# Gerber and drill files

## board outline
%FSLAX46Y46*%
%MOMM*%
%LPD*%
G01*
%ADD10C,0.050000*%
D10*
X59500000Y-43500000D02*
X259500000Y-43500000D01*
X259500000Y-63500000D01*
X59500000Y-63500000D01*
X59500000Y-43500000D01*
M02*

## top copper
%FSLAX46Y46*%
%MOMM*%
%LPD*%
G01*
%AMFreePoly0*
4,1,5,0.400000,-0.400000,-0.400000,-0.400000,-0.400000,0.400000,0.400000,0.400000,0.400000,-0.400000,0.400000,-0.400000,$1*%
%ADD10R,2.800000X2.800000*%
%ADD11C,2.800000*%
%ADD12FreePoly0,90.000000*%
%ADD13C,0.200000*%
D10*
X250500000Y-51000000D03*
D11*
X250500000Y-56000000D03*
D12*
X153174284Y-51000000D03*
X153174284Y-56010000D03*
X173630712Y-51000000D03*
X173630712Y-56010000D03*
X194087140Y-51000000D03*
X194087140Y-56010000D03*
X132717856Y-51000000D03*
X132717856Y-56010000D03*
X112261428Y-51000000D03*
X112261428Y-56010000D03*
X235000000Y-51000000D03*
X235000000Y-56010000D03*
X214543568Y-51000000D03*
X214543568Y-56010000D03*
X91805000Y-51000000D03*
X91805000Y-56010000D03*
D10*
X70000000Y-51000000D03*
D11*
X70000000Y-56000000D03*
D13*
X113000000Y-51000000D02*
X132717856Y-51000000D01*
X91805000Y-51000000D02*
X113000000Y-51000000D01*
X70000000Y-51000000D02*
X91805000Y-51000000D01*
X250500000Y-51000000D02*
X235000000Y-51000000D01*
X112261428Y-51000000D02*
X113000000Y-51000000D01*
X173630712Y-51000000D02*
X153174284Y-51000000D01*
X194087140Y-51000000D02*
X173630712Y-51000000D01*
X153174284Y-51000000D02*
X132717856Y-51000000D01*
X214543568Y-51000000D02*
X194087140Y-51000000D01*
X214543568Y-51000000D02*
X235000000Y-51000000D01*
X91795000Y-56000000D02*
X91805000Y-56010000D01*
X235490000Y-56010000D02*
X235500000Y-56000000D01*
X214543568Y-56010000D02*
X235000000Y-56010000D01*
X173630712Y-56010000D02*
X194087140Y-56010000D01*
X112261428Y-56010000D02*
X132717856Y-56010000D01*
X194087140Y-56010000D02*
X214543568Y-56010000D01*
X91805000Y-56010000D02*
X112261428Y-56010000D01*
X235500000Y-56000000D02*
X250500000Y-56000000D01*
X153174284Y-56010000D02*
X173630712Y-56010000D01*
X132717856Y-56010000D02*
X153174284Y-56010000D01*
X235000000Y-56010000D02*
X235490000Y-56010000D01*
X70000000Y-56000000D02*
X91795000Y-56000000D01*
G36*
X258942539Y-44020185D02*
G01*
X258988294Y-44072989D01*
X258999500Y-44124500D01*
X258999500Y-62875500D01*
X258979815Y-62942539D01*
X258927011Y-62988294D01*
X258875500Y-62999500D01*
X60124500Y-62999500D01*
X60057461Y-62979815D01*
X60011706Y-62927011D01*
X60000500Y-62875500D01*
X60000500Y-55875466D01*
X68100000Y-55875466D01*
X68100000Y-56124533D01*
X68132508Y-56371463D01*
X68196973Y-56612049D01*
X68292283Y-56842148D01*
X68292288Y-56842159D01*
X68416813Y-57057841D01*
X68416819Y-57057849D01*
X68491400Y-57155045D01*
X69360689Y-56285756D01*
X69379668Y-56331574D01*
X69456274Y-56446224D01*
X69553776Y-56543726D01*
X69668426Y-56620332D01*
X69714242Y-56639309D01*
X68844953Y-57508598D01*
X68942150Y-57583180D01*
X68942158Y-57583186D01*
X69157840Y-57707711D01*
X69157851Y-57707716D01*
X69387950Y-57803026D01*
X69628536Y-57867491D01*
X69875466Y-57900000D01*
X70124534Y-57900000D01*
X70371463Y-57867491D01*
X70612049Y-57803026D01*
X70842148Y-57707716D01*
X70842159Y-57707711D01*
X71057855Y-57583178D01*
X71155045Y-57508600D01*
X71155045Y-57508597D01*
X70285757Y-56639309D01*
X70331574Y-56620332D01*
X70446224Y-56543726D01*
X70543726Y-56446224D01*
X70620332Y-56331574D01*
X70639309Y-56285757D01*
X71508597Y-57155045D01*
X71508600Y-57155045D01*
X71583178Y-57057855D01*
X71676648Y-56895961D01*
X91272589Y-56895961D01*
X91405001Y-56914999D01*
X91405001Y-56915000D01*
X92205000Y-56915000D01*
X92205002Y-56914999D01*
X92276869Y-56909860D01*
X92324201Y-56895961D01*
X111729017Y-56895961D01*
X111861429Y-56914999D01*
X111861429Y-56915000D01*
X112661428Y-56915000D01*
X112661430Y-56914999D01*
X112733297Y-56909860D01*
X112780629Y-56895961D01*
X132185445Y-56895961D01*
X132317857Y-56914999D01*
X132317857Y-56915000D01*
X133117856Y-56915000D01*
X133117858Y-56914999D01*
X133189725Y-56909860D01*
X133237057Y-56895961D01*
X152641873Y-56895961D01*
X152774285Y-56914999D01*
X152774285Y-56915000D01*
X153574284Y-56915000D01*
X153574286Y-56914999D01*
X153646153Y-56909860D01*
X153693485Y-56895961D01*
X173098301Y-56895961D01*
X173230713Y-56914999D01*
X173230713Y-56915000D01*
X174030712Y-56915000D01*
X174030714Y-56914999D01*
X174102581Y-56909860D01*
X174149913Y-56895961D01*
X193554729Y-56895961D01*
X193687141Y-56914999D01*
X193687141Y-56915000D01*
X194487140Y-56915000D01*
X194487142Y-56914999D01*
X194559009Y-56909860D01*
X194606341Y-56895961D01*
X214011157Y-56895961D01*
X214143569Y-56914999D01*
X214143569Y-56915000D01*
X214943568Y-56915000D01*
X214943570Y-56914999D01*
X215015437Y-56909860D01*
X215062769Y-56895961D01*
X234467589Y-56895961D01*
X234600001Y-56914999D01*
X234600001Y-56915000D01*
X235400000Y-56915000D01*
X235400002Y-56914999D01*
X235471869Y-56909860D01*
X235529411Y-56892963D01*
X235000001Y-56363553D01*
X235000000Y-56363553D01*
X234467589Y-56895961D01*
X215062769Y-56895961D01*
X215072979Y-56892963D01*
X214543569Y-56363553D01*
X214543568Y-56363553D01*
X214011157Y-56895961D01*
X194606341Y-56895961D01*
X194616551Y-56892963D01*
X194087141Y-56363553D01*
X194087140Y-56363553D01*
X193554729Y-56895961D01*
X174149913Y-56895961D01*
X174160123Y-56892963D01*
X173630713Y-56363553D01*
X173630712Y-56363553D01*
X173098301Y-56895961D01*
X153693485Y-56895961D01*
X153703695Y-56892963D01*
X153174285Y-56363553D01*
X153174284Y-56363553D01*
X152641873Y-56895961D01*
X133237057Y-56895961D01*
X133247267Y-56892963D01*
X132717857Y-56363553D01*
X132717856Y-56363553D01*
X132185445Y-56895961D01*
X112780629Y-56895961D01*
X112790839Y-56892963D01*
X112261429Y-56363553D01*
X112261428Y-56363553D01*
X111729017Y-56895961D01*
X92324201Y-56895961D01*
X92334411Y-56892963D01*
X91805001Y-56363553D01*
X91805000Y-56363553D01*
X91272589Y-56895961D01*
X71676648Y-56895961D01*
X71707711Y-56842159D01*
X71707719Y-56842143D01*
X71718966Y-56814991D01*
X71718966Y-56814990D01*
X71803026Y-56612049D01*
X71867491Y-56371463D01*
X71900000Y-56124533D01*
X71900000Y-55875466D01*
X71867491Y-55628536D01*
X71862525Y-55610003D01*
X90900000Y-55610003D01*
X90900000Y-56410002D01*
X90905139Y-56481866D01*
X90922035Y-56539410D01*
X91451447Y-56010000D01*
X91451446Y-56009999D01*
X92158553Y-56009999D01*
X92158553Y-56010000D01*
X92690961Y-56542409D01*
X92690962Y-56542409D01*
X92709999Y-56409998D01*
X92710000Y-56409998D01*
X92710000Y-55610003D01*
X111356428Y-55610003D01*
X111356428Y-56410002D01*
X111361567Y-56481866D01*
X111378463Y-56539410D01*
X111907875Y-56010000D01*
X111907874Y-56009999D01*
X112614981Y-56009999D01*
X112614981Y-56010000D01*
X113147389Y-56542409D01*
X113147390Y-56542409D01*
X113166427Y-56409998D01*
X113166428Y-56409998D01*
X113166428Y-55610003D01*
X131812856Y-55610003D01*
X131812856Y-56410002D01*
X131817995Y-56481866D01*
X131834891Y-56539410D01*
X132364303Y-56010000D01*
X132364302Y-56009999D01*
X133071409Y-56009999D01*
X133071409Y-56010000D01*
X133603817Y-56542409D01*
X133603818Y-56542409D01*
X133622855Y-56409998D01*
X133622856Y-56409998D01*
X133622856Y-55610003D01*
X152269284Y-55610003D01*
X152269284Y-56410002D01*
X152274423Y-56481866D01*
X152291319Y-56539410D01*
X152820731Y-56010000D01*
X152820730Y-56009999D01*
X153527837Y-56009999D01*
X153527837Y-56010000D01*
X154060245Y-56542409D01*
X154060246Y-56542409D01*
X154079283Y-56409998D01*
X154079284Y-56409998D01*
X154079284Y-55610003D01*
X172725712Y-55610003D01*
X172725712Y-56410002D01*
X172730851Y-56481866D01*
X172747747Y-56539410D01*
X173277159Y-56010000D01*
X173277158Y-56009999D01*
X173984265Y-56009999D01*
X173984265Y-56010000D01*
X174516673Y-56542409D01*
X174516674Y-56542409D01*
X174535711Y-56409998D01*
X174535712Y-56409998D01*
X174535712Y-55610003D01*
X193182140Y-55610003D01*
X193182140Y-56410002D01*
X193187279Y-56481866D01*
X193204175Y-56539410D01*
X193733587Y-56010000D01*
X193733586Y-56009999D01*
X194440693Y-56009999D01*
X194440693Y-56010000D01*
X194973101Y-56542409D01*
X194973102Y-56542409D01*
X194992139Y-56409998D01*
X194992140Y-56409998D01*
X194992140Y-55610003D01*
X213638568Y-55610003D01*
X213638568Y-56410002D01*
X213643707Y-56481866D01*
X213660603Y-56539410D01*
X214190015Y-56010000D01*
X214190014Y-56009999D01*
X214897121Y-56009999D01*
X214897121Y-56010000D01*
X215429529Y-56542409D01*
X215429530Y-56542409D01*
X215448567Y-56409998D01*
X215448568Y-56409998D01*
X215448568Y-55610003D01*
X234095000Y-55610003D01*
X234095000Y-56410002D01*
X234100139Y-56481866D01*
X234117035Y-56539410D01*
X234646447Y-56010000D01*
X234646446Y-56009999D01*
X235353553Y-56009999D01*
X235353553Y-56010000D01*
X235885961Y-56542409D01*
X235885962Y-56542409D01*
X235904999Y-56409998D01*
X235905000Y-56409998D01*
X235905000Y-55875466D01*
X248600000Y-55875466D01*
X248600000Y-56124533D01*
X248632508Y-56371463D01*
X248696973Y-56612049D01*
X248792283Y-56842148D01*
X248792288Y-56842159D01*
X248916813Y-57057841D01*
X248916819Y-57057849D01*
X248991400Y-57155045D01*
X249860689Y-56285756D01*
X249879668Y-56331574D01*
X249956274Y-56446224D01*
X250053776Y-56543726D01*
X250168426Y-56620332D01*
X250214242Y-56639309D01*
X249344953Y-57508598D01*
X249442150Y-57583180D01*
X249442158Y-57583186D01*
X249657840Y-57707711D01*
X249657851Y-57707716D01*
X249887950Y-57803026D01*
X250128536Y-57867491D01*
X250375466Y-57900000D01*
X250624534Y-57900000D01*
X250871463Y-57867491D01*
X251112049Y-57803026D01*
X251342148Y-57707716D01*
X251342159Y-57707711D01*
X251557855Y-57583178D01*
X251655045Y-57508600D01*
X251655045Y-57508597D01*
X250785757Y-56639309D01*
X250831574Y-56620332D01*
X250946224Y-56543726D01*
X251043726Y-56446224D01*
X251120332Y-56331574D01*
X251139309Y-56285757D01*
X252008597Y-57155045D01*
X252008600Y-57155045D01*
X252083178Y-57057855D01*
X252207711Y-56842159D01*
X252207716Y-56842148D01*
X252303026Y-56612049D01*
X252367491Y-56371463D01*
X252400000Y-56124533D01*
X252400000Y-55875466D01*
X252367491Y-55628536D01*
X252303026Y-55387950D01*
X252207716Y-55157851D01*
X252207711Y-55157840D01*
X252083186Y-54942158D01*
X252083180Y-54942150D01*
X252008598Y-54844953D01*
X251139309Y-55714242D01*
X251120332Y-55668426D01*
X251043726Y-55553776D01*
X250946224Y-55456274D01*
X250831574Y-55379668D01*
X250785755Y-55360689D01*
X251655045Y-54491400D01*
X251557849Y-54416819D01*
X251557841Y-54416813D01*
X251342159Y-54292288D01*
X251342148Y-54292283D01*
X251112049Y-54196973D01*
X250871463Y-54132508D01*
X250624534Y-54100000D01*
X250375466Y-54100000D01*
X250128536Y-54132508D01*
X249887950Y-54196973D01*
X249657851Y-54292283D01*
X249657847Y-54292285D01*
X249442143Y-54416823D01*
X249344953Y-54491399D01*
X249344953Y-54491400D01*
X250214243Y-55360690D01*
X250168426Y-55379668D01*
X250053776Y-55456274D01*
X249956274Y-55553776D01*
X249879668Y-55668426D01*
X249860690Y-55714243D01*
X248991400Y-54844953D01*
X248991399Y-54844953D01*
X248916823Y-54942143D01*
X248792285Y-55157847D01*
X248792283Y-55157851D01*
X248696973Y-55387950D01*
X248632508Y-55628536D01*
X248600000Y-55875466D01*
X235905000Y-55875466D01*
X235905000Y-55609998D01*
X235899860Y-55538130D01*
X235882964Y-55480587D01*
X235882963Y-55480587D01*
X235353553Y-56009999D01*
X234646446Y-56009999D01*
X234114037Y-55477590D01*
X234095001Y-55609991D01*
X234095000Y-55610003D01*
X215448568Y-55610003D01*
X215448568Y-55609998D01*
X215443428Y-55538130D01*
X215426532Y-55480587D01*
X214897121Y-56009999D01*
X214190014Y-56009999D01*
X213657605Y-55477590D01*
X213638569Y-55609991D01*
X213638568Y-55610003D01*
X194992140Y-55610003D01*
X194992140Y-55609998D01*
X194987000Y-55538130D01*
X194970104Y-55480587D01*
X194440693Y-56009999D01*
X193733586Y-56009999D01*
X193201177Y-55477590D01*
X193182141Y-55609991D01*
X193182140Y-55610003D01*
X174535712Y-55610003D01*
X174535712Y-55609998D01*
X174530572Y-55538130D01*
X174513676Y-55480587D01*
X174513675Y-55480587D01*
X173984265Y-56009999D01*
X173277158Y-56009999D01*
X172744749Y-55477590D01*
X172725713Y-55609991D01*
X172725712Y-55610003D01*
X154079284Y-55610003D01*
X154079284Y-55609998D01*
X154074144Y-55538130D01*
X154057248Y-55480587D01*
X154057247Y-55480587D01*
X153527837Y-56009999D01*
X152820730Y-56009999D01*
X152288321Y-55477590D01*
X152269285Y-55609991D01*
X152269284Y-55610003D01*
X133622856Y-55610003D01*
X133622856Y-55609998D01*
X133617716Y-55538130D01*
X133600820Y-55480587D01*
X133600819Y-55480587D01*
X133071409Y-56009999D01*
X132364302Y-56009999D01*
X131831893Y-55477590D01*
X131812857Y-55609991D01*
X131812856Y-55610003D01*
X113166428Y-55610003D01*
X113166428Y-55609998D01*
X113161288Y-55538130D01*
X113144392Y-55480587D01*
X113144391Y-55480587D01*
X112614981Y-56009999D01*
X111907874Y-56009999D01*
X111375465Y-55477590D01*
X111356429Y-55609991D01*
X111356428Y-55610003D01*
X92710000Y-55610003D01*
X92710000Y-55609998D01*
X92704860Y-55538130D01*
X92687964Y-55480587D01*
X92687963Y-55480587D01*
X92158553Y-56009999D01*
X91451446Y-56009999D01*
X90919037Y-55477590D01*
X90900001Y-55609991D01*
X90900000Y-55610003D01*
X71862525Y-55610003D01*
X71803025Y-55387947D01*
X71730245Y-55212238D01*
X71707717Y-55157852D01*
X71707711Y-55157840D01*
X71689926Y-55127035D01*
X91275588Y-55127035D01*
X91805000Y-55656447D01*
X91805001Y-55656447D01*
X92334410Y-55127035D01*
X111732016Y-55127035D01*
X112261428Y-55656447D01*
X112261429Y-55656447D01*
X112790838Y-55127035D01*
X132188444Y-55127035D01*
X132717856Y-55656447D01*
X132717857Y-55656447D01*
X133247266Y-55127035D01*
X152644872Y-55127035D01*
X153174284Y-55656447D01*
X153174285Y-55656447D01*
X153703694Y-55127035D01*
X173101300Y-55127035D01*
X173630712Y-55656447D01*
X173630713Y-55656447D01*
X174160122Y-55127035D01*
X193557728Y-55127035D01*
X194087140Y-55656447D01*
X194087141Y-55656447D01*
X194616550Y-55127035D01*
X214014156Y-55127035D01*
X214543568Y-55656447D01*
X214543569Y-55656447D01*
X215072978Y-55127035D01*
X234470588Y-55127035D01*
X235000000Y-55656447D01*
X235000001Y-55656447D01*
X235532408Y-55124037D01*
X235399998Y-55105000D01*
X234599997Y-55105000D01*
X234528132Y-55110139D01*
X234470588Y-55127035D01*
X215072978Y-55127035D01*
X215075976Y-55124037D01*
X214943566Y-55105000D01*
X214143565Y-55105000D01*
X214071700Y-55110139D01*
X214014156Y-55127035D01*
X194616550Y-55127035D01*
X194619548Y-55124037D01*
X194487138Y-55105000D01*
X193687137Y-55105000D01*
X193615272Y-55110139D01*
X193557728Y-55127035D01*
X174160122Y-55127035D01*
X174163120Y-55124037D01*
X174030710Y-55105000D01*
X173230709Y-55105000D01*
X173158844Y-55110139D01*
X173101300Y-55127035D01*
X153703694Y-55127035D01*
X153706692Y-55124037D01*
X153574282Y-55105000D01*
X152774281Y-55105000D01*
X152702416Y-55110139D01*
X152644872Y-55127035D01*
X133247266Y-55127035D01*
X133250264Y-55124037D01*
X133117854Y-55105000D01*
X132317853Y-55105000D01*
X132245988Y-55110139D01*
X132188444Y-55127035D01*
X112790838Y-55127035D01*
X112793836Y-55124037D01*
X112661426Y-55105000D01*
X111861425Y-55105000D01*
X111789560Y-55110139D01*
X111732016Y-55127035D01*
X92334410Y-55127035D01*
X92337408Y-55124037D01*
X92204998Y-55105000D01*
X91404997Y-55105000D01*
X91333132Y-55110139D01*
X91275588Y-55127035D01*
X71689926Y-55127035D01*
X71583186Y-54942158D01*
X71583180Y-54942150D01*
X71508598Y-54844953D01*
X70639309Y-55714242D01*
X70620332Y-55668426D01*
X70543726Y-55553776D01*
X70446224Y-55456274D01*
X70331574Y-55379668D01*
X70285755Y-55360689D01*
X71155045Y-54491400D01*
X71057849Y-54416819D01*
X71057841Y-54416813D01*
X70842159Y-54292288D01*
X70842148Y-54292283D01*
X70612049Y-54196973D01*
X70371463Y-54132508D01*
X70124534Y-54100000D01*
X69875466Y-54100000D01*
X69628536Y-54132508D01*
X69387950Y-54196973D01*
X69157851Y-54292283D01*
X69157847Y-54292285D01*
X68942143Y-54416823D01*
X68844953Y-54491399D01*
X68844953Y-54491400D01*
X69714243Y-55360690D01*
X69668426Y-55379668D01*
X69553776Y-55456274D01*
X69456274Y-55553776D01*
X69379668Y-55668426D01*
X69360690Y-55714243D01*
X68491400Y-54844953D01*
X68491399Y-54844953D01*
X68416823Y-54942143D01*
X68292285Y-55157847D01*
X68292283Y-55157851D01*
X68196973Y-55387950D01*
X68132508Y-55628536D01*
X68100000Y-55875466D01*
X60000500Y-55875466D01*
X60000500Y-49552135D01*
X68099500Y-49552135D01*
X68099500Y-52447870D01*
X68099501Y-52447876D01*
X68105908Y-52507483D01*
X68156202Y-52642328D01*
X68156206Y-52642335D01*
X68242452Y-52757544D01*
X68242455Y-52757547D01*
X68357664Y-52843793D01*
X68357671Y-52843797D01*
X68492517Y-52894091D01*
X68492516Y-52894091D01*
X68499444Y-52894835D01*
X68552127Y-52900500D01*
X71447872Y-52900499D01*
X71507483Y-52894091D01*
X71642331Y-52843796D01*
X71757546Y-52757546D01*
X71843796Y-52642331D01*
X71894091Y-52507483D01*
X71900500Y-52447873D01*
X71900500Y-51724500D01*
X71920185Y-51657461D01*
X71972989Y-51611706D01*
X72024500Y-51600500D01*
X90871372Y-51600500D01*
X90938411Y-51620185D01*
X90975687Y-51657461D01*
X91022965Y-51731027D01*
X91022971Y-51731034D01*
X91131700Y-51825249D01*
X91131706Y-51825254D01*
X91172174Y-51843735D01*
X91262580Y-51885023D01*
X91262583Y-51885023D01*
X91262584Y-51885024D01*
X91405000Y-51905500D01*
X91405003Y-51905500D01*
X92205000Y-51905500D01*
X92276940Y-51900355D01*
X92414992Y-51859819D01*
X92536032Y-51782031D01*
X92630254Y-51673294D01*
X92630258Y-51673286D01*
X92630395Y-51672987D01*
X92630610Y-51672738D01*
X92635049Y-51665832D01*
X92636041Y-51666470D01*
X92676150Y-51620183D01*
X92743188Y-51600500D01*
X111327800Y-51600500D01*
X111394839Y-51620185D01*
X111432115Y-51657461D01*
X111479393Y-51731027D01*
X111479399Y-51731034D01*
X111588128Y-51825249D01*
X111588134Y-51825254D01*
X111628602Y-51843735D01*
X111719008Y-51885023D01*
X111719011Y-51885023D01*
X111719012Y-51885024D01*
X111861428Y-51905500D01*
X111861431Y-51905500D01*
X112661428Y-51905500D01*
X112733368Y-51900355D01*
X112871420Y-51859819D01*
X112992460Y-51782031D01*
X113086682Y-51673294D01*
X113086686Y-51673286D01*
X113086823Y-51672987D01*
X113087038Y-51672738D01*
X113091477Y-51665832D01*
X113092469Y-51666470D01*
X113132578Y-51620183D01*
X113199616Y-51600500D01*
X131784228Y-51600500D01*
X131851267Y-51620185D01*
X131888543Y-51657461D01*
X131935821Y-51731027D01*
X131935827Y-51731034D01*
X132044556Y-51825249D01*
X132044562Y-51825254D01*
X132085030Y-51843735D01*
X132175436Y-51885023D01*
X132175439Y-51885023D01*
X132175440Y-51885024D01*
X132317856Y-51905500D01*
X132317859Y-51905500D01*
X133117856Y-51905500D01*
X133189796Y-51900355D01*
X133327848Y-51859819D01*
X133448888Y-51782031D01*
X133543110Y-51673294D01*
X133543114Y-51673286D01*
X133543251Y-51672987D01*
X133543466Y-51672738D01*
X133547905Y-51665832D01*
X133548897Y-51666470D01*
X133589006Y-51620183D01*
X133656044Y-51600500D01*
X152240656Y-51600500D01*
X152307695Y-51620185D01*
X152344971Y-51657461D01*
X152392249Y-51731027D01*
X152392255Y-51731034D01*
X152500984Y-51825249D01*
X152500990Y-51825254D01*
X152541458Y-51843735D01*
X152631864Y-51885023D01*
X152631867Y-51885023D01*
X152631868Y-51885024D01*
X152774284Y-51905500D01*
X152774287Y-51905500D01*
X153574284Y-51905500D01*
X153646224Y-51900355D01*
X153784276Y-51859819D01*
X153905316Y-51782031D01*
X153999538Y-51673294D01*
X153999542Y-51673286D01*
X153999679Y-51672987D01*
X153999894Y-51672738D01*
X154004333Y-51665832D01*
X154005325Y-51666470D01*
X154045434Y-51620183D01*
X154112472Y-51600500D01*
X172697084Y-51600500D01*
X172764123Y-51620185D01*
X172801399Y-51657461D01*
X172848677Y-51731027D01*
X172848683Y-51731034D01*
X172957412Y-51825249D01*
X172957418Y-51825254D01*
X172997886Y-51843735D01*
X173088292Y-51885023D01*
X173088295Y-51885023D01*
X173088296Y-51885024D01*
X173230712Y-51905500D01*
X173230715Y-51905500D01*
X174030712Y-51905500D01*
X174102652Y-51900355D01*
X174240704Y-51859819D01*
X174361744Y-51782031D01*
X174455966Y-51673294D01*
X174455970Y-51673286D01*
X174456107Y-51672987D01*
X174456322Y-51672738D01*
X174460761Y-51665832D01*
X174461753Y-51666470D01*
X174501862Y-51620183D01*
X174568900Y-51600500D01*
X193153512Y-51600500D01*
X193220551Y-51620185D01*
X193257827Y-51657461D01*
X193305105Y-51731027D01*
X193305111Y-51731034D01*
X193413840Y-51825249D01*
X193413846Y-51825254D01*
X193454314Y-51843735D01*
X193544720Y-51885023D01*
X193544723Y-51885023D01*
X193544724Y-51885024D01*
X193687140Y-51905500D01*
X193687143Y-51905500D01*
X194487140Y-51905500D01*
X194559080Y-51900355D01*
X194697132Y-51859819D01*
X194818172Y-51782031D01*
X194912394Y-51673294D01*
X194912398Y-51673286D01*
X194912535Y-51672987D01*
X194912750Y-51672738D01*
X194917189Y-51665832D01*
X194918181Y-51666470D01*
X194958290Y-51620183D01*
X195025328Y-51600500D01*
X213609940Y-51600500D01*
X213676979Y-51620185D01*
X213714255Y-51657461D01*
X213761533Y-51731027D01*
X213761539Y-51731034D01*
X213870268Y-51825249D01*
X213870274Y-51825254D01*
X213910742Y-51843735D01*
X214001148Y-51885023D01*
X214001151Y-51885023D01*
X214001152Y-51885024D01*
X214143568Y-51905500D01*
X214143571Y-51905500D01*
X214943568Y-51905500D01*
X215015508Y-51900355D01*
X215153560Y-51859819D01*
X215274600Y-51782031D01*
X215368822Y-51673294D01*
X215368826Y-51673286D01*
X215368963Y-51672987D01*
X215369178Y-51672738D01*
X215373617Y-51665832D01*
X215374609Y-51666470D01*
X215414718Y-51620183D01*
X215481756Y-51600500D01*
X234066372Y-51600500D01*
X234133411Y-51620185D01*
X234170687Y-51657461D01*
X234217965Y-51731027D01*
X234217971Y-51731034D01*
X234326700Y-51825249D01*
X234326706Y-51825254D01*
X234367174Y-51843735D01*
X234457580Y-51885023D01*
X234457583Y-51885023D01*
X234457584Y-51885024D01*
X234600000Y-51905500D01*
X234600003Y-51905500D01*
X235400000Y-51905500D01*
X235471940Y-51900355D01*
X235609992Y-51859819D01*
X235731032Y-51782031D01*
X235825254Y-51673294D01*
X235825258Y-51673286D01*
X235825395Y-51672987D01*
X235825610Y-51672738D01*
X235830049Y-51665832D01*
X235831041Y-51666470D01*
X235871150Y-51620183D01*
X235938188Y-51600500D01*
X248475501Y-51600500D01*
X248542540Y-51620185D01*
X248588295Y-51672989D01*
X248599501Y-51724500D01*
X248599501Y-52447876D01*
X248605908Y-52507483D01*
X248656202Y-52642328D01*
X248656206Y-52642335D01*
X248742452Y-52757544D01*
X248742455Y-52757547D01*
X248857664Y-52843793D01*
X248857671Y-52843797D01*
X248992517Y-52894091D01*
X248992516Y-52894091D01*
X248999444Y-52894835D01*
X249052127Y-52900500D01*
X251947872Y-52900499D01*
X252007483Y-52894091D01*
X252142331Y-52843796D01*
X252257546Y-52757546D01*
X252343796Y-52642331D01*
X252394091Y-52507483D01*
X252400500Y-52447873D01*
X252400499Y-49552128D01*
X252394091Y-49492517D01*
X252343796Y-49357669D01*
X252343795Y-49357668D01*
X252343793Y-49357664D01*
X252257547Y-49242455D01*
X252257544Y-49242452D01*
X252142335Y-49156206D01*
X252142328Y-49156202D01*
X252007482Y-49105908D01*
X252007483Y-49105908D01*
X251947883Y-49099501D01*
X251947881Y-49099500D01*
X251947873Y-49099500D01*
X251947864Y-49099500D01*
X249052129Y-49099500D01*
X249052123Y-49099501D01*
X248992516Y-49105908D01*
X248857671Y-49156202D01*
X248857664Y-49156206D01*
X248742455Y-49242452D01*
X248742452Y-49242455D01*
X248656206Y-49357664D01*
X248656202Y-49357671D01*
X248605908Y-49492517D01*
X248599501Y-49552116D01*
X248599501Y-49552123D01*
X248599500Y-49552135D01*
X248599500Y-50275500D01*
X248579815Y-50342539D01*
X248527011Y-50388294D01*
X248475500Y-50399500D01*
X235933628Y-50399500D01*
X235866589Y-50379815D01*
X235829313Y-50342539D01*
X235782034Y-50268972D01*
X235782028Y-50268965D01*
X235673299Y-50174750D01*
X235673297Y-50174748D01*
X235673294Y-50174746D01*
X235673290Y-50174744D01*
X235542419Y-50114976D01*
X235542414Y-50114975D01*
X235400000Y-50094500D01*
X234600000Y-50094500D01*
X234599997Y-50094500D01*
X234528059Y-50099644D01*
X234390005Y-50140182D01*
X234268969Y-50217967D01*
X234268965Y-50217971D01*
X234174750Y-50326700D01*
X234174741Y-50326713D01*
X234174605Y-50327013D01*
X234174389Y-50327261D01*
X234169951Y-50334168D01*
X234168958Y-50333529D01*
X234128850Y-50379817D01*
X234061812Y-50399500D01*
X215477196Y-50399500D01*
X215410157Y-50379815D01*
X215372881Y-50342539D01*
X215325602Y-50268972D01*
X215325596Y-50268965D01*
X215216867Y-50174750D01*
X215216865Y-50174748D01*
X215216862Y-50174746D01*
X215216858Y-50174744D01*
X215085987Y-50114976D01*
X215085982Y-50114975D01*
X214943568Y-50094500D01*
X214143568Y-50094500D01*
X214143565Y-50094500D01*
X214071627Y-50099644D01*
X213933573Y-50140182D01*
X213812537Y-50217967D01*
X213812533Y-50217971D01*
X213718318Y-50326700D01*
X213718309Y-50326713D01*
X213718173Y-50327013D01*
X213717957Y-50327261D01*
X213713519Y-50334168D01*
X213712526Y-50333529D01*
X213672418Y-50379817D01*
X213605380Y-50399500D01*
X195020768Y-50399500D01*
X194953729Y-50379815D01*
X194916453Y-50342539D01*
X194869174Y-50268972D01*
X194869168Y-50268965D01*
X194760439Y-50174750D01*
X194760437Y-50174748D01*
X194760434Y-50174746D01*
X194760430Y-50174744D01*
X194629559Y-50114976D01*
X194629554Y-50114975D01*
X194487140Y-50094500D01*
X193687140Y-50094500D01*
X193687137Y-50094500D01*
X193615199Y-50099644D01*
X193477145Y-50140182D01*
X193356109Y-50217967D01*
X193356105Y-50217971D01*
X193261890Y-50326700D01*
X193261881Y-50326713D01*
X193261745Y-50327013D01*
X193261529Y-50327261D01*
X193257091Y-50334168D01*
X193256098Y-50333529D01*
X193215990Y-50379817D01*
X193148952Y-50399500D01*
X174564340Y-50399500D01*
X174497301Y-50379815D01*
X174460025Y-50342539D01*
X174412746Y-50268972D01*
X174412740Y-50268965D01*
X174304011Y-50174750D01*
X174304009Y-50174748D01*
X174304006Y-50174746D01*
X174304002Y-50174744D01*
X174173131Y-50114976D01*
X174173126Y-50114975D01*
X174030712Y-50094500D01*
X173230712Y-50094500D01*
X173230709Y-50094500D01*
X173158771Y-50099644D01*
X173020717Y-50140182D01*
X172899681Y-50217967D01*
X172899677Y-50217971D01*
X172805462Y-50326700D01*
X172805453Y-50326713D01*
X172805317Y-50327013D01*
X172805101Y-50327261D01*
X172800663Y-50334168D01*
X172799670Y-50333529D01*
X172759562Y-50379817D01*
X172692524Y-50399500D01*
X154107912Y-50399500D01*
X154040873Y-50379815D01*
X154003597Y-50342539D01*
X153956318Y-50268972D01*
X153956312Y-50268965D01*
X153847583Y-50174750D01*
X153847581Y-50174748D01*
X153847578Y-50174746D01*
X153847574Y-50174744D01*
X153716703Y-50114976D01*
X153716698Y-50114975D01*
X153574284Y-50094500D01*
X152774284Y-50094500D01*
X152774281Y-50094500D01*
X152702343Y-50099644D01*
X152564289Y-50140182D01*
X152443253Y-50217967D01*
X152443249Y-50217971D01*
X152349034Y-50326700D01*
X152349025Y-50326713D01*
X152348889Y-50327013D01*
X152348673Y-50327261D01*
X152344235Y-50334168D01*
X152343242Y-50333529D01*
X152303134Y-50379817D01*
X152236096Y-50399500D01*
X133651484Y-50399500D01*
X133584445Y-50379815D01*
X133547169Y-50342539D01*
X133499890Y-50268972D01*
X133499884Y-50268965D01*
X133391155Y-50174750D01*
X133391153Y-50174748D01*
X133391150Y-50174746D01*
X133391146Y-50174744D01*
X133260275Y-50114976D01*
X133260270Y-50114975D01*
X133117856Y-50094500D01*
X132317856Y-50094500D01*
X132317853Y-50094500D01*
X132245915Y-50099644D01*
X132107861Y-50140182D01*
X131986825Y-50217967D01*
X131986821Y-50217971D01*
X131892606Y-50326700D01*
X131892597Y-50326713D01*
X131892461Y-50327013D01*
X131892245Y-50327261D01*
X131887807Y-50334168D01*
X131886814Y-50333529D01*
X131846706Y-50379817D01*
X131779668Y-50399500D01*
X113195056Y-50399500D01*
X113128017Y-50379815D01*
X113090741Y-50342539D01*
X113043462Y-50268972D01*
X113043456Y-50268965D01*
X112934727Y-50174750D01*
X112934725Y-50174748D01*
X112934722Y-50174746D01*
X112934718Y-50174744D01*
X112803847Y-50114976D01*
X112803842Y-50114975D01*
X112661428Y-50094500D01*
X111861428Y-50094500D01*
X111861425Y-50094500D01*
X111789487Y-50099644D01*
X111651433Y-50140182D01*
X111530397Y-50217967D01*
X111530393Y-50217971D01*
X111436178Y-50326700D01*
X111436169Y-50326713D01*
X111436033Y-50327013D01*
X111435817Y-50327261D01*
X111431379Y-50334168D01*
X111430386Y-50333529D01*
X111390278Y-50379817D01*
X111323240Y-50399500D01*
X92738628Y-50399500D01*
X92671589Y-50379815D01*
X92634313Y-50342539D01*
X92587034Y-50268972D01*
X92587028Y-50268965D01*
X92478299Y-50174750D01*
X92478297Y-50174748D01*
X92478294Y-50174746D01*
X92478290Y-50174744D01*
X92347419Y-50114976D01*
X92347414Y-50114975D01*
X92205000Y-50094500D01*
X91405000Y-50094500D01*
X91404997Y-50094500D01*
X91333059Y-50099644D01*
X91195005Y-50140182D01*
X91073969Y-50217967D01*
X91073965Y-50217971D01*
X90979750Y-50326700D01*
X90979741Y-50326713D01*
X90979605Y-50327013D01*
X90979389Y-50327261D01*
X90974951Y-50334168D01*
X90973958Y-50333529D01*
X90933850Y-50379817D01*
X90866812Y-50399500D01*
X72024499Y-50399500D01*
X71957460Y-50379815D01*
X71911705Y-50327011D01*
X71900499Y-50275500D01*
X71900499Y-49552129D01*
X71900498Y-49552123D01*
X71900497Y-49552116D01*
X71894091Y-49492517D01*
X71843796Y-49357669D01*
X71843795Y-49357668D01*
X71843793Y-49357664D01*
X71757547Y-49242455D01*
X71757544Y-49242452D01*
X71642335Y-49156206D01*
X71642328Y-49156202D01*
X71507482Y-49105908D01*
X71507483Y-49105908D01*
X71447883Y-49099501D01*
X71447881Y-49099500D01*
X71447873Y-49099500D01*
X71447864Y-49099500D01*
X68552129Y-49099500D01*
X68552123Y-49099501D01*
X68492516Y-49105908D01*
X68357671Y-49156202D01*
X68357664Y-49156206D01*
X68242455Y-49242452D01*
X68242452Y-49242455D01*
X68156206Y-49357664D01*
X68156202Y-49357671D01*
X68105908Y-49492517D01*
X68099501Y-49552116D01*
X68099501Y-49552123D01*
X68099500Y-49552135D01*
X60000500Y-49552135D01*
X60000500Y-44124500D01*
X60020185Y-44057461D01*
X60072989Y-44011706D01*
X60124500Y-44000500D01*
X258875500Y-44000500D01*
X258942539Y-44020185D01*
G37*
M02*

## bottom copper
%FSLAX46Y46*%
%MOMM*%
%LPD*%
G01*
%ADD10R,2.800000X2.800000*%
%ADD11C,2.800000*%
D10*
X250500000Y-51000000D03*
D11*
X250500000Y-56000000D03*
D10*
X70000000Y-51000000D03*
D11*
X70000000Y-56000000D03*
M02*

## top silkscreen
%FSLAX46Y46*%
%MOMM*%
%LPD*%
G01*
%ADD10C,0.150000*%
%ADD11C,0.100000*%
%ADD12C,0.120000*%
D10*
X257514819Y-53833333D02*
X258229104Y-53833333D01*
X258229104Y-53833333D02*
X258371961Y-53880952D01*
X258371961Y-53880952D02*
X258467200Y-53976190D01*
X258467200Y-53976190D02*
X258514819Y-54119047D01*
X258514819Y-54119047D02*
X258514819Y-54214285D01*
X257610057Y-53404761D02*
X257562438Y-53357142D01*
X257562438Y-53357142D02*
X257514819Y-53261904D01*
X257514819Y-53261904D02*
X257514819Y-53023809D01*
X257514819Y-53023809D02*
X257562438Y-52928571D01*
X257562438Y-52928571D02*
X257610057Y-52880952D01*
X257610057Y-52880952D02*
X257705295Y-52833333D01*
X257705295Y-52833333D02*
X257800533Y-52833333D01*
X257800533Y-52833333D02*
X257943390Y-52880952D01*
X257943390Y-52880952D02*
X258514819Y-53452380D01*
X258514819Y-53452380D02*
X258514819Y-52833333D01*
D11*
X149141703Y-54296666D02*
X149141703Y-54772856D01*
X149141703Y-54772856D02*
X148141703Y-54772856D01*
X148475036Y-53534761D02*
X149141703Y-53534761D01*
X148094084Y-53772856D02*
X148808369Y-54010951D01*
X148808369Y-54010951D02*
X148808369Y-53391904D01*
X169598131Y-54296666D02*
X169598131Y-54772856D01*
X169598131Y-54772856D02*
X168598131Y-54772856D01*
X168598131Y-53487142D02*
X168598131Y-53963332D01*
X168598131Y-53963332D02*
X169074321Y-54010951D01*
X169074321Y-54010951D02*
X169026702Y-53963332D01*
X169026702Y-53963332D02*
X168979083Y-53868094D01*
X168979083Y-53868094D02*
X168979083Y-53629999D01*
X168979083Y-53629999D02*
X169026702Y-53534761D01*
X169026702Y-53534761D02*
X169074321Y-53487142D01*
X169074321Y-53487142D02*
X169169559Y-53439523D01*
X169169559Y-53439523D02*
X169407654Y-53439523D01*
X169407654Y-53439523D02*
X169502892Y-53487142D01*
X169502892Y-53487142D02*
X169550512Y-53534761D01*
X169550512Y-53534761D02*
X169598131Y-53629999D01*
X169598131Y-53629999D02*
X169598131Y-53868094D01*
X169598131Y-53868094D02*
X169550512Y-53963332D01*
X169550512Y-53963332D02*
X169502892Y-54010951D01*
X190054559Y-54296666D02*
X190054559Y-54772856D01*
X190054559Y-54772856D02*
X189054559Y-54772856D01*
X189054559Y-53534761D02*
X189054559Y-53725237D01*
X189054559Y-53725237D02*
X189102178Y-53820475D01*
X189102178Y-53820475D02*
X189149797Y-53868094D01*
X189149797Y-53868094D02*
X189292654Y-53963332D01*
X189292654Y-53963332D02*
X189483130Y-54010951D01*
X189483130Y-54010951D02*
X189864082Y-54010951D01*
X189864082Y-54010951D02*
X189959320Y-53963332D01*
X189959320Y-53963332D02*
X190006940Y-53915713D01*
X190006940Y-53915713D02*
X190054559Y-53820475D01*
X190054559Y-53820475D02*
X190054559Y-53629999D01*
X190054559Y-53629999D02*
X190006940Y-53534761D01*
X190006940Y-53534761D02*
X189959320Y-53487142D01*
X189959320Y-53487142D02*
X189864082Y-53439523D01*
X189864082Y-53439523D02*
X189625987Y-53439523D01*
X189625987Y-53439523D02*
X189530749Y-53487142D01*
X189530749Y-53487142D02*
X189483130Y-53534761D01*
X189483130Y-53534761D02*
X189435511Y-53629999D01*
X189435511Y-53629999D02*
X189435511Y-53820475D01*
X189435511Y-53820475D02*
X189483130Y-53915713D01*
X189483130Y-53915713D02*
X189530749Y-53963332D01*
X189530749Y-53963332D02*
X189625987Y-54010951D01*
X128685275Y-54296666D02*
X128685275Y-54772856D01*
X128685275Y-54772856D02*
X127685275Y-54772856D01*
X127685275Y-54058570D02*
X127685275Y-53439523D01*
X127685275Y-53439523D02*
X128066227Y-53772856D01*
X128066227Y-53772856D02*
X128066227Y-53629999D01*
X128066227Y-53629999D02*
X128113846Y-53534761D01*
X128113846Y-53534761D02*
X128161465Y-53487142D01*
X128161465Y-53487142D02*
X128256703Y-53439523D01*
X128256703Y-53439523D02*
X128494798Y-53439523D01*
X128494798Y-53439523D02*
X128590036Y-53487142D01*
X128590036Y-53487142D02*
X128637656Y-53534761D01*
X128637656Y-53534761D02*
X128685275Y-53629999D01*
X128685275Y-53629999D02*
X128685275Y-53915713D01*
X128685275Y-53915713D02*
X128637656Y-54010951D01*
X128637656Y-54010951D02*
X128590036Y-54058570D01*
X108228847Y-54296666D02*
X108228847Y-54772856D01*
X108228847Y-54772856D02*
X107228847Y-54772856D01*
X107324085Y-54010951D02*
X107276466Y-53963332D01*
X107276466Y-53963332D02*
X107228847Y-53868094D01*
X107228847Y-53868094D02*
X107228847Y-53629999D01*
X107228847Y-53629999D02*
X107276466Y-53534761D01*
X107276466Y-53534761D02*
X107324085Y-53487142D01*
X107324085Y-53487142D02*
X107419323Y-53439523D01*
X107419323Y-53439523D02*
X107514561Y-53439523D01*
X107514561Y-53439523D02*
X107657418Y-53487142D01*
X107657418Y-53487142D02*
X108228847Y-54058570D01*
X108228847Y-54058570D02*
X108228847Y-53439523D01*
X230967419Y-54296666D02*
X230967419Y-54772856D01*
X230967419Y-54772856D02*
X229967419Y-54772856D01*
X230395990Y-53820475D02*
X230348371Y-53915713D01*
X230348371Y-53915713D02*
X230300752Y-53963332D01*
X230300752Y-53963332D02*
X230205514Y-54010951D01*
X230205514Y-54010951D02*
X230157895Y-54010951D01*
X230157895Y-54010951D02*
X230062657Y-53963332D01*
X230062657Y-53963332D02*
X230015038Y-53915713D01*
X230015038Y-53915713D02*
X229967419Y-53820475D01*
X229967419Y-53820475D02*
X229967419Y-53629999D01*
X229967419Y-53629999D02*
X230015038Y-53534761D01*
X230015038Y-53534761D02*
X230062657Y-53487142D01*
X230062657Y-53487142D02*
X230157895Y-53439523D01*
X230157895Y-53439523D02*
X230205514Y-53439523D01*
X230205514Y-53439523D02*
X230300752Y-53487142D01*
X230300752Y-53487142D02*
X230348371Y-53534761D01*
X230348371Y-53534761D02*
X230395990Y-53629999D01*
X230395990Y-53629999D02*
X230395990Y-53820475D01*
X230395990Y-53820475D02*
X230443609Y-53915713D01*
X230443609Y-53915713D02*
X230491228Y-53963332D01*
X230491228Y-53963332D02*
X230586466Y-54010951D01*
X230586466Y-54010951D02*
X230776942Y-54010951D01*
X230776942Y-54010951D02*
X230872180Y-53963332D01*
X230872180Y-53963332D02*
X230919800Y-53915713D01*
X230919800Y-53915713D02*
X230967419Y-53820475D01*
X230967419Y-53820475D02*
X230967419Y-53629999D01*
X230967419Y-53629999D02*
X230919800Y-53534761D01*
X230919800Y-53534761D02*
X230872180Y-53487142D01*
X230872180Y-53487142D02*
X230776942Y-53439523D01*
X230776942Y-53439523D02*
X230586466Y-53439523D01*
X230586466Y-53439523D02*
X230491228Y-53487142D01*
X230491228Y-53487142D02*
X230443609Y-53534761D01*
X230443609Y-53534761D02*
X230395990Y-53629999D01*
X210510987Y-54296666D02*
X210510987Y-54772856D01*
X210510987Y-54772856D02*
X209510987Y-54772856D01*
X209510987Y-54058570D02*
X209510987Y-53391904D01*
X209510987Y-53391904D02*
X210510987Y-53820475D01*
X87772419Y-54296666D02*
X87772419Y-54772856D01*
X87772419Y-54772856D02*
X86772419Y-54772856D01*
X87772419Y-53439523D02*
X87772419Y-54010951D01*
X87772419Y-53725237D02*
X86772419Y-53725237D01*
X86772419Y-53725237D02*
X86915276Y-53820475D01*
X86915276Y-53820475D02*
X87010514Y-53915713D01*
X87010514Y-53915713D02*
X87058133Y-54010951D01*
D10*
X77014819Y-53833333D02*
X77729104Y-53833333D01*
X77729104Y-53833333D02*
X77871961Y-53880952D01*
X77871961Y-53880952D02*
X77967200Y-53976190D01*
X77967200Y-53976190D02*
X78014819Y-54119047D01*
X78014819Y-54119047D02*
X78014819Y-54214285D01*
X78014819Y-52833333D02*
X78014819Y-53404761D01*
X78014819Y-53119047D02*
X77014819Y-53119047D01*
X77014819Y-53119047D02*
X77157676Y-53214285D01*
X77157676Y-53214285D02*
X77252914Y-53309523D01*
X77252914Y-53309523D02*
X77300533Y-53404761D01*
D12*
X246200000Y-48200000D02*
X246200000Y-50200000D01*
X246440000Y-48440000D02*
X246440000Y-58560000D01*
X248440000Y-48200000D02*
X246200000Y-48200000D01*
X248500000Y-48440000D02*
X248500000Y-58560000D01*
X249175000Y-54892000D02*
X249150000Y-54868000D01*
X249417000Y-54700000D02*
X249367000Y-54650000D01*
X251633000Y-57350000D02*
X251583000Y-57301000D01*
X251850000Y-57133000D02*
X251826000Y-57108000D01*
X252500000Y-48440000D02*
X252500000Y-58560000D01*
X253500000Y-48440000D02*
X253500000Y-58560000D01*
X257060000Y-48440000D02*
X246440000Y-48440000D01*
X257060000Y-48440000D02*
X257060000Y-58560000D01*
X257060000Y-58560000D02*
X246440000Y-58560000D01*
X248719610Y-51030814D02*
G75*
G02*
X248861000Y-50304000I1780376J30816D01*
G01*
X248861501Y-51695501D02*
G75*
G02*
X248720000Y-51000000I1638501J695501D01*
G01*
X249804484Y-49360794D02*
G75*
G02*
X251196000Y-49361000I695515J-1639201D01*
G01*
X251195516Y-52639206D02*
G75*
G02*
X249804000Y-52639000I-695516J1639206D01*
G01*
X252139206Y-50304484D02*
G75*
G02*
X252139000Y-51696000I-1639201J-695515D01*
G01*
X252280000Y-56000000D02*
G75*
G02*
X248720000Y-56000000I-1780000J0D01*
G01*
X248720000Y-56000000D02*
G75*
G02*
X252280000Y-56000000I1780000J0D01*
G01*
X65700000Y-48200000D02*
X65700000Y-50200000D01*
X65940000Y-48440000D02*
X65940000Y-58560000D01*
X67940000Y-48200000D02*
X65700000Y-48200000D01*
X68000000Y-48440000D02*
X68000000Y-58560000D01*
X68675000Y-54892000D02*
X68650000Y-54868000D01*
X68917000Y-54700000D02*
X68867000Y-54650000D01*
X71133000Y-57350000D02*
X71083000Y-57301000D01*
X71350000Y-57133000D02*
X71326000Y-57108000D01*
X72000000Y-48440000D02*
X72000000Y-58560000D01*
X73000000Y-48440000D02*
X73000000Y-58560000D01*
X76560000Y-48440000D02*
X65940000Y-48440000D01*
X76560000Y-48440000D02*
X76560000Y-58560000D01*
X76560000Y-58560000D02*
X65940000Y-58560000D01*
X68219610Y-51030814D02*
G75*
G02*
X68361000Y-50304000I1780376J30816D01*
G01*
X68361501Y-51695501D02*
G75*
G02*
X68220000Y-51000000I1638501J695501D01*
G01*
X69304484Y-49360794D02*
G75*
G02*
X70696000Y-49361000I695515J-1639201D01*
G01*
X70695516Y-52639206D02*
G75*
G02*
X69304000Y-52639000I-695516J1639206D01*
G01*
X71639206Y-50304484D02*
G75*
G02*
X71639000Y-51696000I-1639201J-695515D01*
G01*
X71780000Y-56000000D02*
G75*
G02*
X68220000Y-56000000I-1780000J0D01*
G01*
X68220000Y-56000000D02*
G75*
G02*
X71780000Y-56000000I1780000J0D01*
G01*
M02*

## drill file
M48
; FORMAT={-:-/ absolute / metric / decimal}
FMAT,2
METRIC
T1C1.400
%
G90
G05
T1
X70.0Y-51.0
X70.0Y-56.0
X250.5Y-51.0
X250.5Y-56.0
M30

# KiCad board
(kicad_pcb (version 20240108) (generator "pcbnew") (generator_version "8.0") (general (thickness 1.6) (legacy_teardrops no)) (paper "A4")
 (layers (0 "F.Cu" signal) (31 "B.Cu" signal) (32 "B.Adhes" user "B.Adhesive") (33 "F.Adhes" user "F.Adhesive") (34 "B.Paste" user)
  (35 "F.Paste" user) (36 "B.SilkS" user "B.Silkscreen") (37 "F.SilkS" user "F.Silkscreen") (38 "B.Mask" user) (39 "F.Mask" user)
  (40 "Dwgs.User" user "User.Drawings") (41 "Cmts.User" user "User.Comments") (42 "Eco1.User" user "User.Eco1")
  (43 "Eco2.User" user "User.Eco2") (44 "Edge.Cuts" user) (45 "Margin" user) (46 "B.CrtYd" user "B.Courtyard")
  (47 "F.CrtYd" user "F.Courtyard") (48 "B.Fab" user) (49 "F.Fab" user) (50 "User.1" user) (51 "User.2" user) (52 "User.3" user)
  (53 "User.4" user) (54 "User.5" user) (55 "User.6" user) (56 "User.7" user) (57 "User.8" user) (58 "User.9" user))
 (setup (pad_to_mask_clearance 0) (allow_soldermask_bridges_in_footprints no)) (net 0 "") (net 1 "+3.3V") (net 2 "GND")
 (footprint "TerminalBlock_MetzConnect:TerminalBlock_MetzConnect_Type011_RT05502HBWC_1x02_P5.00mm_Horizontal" (layer "F.Cu")
  (at 250.5 51 -90)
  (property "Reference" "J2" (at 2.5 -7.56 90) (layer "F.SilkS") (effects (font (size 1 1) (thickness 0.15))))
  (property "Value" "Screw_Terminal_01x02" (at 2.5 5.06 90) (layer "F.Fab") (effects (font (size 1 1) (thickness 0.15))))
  (fp_line (start -2.8 4.3) (end -0.8 4.3) (stroke (width 0.12) (type solid)) (layer "F.SilkS"))
  (fp_line (start -2.56 4.06) (end 7.56 4.06) (stroke (width 0.12) (type solid)) (layer "F.SilkS"))
  (fp_line (start -2.8 2.06) (end -2.8 4.3) (stroke (width 0.12) (type solid)) (layer "F.SilkS"))
  (fp_line (start -2.56 2) (end 7.56 2) (stroke (width 0.12) (type solid)) (layer "F.SilkS"))
  (fp_line (start 3.892 1.325) (end 3.868 1.35) (stroke (width 0.12) (type solid)) (layer "F.SilkS"))
  (fp_line (start 3.7 1.083) (end 3.65 1.133) (stroke (width 0.12) (type solid)) (layer "F.SilkS"))
  (fp_line (start 6.35 -1.133) (end 6.301 -1.083) (stroke (width 0.12) (type solid)) (layer "F.SilkS"))
  (fp_line (start 6.133 -1.35) (end 6.108 -1.326) (stroke (width 0.12) (type solid)) (layer "F.SilkS"))
  (fp_line (start -2.56 -2) (end 7.56 -2) (stroke (width 0.12) (type solid)) (layer "F.SilkS"))
  (fp_line (start -2.56 -3) (end 7.56 -3) (stroke (width 0.12) (type solid)) (layer "F.SilkS"))
  (fp_line (start -2.56 -6.56) (end -2.56 4.06) (stroke (width 0.12) (type solid)) (layer "F.SilkS"))
  (fp_line (start -2.56 -6.56) (end 7.56 -6.56) (stroke (width 0.12) (type solid)) (layer "F.SilkS"))
  (fp_line (start 7.56 -6.56) (end 7.56 4.06) (stroke (width 0.12) (type solid)) (layer "F.SilkS"))
  (fp_arc (start 0.030814 1.78039) (mid -0.340023 1.747891) (end -0.696 1.639) (stroke (width 0.12) (type solid)) (layer "F.SilkS"))
  (fp_arc (start 0.695501 1.638499) (mid 0.354875 1.744266) (end 0 1.78) (stroke (width 0.12) (type solid)) (layer "F.SilkS"))
  (fp_arc (start -1.639206 0.695516) (mid -1.780657 -0.000263) (end -1.639 -0.696) (stroke (width 0.12) (type solid)) (layer "F.SilkS"))
  (fp_arc (start 1.639206 -0.695516) (mid 1.780657 0.000263) (end 1.639 0.696) (stroke (width 0.12) (type solid)) (layer "F.SilkS"))
  (fp_arc (start -0.695516 -1.639206) (mid 0.000263 -1.780657) (end 0.696 -1.639) (stroke (width 0.12) (type solid)) (layer "F.SilkS"))
  (fp_circle (center 5 0) (end 6.78 0) (stroke (width 0.12) (type solid)) (fill none) (layer "F.SilkS"))
  (pad "1" thru_hole rect (at 0 0 270) (size 2.8 2.8) (drill 1.4) (layers "*.Cu" "*.Mask") (remove_unused_layers no) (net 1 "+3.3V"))
  (pad "2" thru_hole circle (at 5 0 270) (size 2.8 2.8) (drill 1.4) (layers "*.Cu" "*.Mask") (remove_unused_layers no) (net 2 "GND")))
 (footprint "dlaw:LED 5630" (layer "F.Cu") (at 153.864284 54.31 90)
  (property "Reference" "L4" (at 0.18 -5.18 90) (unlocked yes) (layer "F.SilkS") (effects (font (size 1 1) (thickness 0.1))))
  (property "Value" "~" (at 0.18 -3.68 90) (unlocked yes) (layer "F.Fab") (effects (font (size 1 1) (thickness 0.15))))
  (pad "1" smd custom (at 3.31 -0.69 90) (size 0.8 0.8) (layers "F.Cu" "F.Paste" "F.Mask") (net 1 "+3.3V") (thermal_bridge_angle 45)
   (options (clearance outline) (anchor rect)) (primitives))
  (pad "3" smd custom (at -1.7 -0.69 90) (size 0.8 0.8) (layers "F.Cu" "F.Paste" "F.Mask") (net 2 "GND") (thermal_bridge_angle 45)
   (options (clearance outline) (anchor rect)) (primitives)))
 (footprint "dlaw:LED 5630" (layer "F.Cu") (at 174.320712 54.31 90)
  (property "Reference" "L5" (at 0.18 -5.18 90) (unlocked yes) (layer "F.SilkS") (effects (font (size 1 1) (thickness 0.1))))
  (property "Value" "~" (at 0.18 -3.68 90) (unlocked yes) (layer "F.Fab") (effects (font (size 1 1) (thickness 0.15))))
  (pad "1" smd custom (at 3.31 -0.69 90) (size 0.8 0.8) (layers "F.Cu" "F.Paste" "F.Mask") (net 1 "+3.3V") (thermal_bridge_angle 45)
   (options (clearance outline) (anchor rect)) (primitives))
  (pad "3" smd custom (at -1.7 -0.69 90) (size 0.8 0.8) (layers "F.Cu" "F.Paste" "F.Mask") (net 2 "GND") (thermal_bridge_angle 45)
   (options (clearance outline) (anchor rect)) (primitives)))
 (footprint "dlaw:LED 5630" (layer "F.Cu") (at 194.77714 54.31 90)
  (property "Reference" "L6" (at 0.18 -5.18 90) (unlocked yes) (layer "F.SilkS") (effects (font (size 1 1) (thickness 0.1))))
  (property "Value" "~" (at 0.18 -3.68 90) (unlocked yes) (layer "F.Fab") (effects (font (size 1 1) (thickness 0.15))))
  (pad "1" smd custom (at 3.31 -0.69 90) (size 0.8 0.8) (layers "F.Cu" "F.Paste" "F.Mask") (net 1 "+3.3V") (thermal_bridge_angle 45)
   (options (clearance outline) (anchor rect)) (primitives))
  (pad "3" smd custom (at -1.7 -0.69 90) (size 0.8 0.8) (layers "F.Cu" "F.Paste" "F.Mask") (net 2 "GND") (thermal_bridge_angle 45)
   (options (clearance outline) (anchor rect)) (primitives)))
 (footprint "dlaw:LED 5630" (layer "F.Cu") (at 133.407856 54.31 90)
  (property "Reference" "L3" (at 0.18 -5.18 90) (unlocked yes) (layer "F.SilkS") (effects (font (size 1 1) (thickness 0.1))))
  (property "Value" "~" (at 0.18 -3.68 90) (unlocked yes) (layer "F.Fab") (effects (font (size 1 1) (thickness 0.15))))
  (pad "1" smd custom (at 3.31 -0.69 90) (size 0.8 0.8) (layers "F.Cu" "F.Paste" "F.Mask") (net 1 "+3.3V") (thermal_bridge_angle 45)
   (options (clearance outline) (anchor rect)) (primitives))
  (pad "3" smd custom (at -1.7 -0.69 90) (size 0.8 0.8) (layers "F.Cu" "F.Paste" "F.Mask") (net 2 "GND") (thermal_bridge_angle 45)
   (options (clearance outline) (anchor rect)) (primitives)))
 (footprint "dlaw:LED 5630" (layer "F.Cu") (at 112.951428 54.31 90)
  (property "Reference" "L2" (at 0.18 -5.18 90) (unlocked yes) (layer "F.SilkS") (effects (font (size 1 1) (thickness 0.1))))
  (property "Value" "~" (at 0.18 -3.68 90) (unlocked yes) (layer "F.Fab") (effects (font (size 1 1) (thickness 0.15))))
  (pad "1" smd custom (at 3.31 -0.69 90) (size 0.8 0.8) (layers "F.Cu" "F.Paste" "F.Mask") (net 1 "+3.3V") (thermal_bridge_angle 45)
   (options (clearance outline) (anchor rect)) (primitives))
  (pad "3" smd custom (at -1.7 -0.69 90) (size 0.8 0.8) (layers "F.Cu" "F.Paste" "F.Mask") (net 2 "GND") (thermal_bridge_angle 45)
   (options (clearance outline) (anchor rect)) (primitives)))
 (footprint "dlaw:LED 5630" (layer "F.Cu") (at 235.69 54.31 90)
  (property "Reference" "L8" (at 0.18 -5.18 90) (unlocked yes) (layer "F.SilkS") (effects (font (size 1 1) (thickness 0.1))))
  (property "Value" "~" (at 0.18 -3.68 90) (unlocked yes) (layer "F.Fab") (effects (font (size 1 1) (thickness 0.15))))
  (pad "1" smd custom (at 3.31 -0.69 90) (size 0.8 0.8) (layers "F.Cu" "F.Paste" "F.Mask") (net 1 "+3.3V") (thermal_bridge_angle 45)
   (options (clearance outline) (anchor rect)) (primitives))
  (pad "3" smd custom (at -1.7 -0.69 90) (size 0.8 0.8) (layers "F.Cu" "F.Paste" "F.Mask") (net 2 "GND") (thermal_bridge_angle 45)
   (options (clearance outline) (anchor rect)) (primitives)))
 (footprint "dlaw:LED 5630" (layer "F.Cu") (at 215.233568 54.31 90)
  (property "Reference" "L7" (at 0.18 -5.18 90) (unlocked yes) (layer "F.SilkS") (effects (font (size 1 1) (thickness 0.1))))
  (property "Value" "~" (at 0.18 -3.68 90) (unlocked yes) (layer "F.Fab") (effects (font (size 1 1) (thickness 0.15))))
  (pad "1" smd custom (at 3.31 -0.69 90) (size 0.8 0.8) (layers "F.Cu" "F.Paste" "F.Mask") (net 1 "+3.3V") (thermal_bridge_angle 45)
   (options (clearance outline) (anchor rect)) (primitives))
  (pad "3" smd custom (at -1.7 -0.69 90) (size 0.8 0.8) (layers "F.Cu" "F.Paste" "F.Mask") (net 2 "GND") (thermal_bridge_angle 45)
   (options (clearance outline) (anchor rect)) (primitives)))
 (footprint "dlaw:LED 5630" (layer "F.Cu") (at 92.495 54.31 90)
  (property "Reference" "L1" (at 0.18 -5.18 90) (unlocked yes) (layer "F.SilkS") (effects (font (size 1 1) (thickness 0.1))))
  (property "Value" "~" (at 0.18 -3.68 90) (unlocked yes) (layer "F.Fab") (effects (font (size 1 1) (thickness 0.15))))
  (pad "1" smd custom (at 3.31 -0.69 90) (size 0.8 0.8) (layers "F.Cu" "F.Paste" "F.Mask") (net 1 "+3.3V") (thermal_bridge_angle 45)
   (options (clearance outline) (anchor rect)) (primitives))
  (pad "3" smd custom (at -1.7 -0.69 90) (size 0.8 0.8) (layers "F.Cu" "F.Paste" "F.Mask") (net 2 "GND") (thermal_bridge_angle 45)
   (options (clearance outline) (anchor rect)) (primitives)))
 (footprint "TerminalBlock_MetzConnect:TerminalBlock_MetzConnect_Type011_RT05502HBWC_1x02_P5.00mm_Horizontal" (layer "F.Cu") (at 70 51 -90)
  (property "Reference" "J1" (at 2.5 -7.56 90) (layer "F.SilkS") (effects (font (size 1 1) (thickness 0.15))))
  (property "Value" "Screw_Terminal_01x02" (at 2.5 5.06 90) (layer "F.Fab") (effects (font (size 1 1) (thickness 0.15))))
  (fp_line (start -2.8 4.3) (end -0.8 4.3) (stroke (width 0.12) (type solid)) (layer "F.SilkS"))
  (fp_line (start -2.56 4.06) (end 7.56 4.06) (stroke (width 0.12) (type solid)) (layer "F.SilkS"))
  (fp_line (start -2.8 2.06) (end -2.8 4.3) (stroke (width 0.12) (type solid)) (layer "F.SilkS"))
  (fp_line (start -2.56 2) (end 7.56 2) (stroke (width 0.12) (type solid)) (layer "F.SilkS"))
  (fp_line (start 3.892 1.325) (end 3.868 1.35) (stroke (width 0.12) (type solid)) (layer "F.SilkS"))
  (fp_line (start 3.7 1.083) (end 3.65 1.133) (stroke (width 0.12) (type solid)) (layer "F.SilkS"))
  (fp_line (start 6.35 -1.133) (end 6.301 -1.083) (stroke (width 0.12) (type solid)) (layer "F.SilkS"))
  (fp_line (start 6.133 -1.35) (end 6.108 -1.326) (stroke (width 0.12) (type solid)) (layer "F.SilkS"))
  (fp_line (start -2.56 -2) (end 7.56 -2) (stroke (width 0.12) (type solid)) (layer "F.SilkS"))
  (fp_line (start -2.56 -3) (end 7.56 -3) (stroke (width 0.12) (type solid)) (layer "F.SilkS"))
  (fp_line (start -2.56 -6.56) (end -2.56 4.06) (stroke (width 0.12) (type solid)) (layer "F.SilkS"))
  (fp_line (start -2.56 -6.56) (end 7.56 -6.56) (stroke (width 0.12) (type solid)) (layer "F.SilkS"))
  (fp_line (start 7.56 -6.56) (end 7.56 4.06) (stroke (width 0.12) (type solid)) (layer "F.SilkS"))
  (fp_arc (start 0.030814 1.78039) (mid -0.340023 1.747891) (end -0.696 1.639) (stroke (width 0.12) (type solid)) (layer "F.SilkS"))
  (fp_arc (start 0.695501 1.638499) (mid 0.354875 1.744266) (end 0 1.78) (stroke (width 0.12) (type solid)) (layer "F.SilkS"))
  (fp_arc (start -1.639206 0.695516) (mid -1.780657 -0.000263) (end -1.639 -0.696) (stroke (width 0.12) (type solid)) (layer "F.SilkS"))
  (fp_arc (start 1.639206 -0.695516) (mid 1.780657 0.000263) (end 1.639 0.696) (stroke (width 0.12) (type solid)) (layer "F.SilkS"))
  (fp_arc (start -0.695516 -1.639206) (mid 0.000263 -1.780657) (end 0.696 -1.639) (stroke (width 0.12) (type solid)) (layer "F.SilkS"))
  (fp_circle (center 5 0) (end 6.78 0) (stroke (width 0.12) (type solid)) (fill none) (layer "F.SilkS"))
  (pad "1" thru_hole rect (at 0 0 270) (size 2.8 2.8) (drill 1.4) (layers "*.Cu" "*.Mask") (remove_unused_layers no) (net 1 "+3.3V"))
  (pad "2" thru_hole circle (at 5 0 270) (size 2.8 2.8) (drill 1.4) (layers "*.Cu" "*.Mask") (remove_unused_layers no) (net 2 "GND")))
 (gr_rect (start 59.5 43.5) (end 259.5 63.5) (stroke (width 0.05) (type default)) (fill none) (layer "Edge.Cuts"))
 (segment (start 113 51) (end 132.717856 51) (width 0.2) (layer "F.Cu") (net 1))
 (segment (start 91.805 51) (end 113 51) (width 0.2) (layer "F.Cu") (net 1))
 (segment (start 70 51) (end 91.805 51) (width 0.2) (layer "F.Cu") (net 1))
 (segment (start 250.5 51) (end 235 51) (width 0.2) (layer "F.Cu") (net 1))
 (segment (start 112.261428 51) (end 113 51) (width 0.2) (layer "F.Cu") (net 1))
 (segment (start 173.630712 51) (end 153.174284 51) (width 0.2) (layer "F.Cu") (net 1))
 (segment (start 194.08714 51) (end 173.630712 51) (width 0.2) (layer "F.Cu") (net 1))
 (segment (start 153.174284 51) (end 132.717856 51) (width 0.2) (layer "F.Cu") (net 1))
 (segment (start 214.543568 51) (end 194.08714 51) (width 0.2) (layer "F.Cu") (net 1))
 (segment (start 214.543568 51) (end 235 51) (width 0.2) (layer "F.Cu") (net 1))
 (segment (start 91.795 56) (end 91.805 56.01) (width 0.2) (layer "F.Cu") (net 2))
 (segment (start 235.49 56.01) (end 235.5 56) (width 0.2) (layer "F.Cu") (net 2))
 (segment (start 214.543568 56.01) (end 235 56.01) (width 0.2) (layer "F.Cu") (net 2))
 (segment (start 173.630712 56.01) (end 194.08714 56.01) (width 0.2) (layer "F.Cu") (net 2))
 (segment (start 112.261428 56.01) (end 132.717856 56.01) (width 0.2) (layer "F.Cu") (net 2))
 (segment (start 194.08714 56.01) (end 214.543568 56.01) (width 0.2) (layer "F.Cu") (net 2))
 (segment (start 91.805 56.01) (end 112.261428 56.01) (width 0.2) (layer "F.Cu") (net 2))
 (segment (start 235.5 56) (end 250.5 56) (width 0.2) (layer "F.Cu") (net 2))
 (segment (start 153.174284 56.01) (end 173.630712 56.01) (width 0.2) (layer "F.Cu") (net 2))
 (segment (start 132.717856 56.01) (end 153.174284 56.01) (width 0.2) (layer "F.Cu") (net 2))
 (segment (start 235 56.01) (end 235.49 56.01) (width 0.2) (layer "F.Cu") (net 2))
 (segment (start 70 56) (end 91.795 56) (width 0.2) (layer "F.Cu") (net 2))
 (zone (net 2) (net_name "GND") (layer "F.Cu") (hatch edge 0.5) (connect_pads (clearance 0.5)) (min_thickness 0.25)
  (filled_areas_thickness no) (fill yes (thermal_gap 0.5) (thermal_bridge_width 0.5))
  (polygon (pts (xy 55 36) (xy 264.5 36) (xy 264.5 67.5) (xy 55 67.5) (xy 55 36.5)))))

